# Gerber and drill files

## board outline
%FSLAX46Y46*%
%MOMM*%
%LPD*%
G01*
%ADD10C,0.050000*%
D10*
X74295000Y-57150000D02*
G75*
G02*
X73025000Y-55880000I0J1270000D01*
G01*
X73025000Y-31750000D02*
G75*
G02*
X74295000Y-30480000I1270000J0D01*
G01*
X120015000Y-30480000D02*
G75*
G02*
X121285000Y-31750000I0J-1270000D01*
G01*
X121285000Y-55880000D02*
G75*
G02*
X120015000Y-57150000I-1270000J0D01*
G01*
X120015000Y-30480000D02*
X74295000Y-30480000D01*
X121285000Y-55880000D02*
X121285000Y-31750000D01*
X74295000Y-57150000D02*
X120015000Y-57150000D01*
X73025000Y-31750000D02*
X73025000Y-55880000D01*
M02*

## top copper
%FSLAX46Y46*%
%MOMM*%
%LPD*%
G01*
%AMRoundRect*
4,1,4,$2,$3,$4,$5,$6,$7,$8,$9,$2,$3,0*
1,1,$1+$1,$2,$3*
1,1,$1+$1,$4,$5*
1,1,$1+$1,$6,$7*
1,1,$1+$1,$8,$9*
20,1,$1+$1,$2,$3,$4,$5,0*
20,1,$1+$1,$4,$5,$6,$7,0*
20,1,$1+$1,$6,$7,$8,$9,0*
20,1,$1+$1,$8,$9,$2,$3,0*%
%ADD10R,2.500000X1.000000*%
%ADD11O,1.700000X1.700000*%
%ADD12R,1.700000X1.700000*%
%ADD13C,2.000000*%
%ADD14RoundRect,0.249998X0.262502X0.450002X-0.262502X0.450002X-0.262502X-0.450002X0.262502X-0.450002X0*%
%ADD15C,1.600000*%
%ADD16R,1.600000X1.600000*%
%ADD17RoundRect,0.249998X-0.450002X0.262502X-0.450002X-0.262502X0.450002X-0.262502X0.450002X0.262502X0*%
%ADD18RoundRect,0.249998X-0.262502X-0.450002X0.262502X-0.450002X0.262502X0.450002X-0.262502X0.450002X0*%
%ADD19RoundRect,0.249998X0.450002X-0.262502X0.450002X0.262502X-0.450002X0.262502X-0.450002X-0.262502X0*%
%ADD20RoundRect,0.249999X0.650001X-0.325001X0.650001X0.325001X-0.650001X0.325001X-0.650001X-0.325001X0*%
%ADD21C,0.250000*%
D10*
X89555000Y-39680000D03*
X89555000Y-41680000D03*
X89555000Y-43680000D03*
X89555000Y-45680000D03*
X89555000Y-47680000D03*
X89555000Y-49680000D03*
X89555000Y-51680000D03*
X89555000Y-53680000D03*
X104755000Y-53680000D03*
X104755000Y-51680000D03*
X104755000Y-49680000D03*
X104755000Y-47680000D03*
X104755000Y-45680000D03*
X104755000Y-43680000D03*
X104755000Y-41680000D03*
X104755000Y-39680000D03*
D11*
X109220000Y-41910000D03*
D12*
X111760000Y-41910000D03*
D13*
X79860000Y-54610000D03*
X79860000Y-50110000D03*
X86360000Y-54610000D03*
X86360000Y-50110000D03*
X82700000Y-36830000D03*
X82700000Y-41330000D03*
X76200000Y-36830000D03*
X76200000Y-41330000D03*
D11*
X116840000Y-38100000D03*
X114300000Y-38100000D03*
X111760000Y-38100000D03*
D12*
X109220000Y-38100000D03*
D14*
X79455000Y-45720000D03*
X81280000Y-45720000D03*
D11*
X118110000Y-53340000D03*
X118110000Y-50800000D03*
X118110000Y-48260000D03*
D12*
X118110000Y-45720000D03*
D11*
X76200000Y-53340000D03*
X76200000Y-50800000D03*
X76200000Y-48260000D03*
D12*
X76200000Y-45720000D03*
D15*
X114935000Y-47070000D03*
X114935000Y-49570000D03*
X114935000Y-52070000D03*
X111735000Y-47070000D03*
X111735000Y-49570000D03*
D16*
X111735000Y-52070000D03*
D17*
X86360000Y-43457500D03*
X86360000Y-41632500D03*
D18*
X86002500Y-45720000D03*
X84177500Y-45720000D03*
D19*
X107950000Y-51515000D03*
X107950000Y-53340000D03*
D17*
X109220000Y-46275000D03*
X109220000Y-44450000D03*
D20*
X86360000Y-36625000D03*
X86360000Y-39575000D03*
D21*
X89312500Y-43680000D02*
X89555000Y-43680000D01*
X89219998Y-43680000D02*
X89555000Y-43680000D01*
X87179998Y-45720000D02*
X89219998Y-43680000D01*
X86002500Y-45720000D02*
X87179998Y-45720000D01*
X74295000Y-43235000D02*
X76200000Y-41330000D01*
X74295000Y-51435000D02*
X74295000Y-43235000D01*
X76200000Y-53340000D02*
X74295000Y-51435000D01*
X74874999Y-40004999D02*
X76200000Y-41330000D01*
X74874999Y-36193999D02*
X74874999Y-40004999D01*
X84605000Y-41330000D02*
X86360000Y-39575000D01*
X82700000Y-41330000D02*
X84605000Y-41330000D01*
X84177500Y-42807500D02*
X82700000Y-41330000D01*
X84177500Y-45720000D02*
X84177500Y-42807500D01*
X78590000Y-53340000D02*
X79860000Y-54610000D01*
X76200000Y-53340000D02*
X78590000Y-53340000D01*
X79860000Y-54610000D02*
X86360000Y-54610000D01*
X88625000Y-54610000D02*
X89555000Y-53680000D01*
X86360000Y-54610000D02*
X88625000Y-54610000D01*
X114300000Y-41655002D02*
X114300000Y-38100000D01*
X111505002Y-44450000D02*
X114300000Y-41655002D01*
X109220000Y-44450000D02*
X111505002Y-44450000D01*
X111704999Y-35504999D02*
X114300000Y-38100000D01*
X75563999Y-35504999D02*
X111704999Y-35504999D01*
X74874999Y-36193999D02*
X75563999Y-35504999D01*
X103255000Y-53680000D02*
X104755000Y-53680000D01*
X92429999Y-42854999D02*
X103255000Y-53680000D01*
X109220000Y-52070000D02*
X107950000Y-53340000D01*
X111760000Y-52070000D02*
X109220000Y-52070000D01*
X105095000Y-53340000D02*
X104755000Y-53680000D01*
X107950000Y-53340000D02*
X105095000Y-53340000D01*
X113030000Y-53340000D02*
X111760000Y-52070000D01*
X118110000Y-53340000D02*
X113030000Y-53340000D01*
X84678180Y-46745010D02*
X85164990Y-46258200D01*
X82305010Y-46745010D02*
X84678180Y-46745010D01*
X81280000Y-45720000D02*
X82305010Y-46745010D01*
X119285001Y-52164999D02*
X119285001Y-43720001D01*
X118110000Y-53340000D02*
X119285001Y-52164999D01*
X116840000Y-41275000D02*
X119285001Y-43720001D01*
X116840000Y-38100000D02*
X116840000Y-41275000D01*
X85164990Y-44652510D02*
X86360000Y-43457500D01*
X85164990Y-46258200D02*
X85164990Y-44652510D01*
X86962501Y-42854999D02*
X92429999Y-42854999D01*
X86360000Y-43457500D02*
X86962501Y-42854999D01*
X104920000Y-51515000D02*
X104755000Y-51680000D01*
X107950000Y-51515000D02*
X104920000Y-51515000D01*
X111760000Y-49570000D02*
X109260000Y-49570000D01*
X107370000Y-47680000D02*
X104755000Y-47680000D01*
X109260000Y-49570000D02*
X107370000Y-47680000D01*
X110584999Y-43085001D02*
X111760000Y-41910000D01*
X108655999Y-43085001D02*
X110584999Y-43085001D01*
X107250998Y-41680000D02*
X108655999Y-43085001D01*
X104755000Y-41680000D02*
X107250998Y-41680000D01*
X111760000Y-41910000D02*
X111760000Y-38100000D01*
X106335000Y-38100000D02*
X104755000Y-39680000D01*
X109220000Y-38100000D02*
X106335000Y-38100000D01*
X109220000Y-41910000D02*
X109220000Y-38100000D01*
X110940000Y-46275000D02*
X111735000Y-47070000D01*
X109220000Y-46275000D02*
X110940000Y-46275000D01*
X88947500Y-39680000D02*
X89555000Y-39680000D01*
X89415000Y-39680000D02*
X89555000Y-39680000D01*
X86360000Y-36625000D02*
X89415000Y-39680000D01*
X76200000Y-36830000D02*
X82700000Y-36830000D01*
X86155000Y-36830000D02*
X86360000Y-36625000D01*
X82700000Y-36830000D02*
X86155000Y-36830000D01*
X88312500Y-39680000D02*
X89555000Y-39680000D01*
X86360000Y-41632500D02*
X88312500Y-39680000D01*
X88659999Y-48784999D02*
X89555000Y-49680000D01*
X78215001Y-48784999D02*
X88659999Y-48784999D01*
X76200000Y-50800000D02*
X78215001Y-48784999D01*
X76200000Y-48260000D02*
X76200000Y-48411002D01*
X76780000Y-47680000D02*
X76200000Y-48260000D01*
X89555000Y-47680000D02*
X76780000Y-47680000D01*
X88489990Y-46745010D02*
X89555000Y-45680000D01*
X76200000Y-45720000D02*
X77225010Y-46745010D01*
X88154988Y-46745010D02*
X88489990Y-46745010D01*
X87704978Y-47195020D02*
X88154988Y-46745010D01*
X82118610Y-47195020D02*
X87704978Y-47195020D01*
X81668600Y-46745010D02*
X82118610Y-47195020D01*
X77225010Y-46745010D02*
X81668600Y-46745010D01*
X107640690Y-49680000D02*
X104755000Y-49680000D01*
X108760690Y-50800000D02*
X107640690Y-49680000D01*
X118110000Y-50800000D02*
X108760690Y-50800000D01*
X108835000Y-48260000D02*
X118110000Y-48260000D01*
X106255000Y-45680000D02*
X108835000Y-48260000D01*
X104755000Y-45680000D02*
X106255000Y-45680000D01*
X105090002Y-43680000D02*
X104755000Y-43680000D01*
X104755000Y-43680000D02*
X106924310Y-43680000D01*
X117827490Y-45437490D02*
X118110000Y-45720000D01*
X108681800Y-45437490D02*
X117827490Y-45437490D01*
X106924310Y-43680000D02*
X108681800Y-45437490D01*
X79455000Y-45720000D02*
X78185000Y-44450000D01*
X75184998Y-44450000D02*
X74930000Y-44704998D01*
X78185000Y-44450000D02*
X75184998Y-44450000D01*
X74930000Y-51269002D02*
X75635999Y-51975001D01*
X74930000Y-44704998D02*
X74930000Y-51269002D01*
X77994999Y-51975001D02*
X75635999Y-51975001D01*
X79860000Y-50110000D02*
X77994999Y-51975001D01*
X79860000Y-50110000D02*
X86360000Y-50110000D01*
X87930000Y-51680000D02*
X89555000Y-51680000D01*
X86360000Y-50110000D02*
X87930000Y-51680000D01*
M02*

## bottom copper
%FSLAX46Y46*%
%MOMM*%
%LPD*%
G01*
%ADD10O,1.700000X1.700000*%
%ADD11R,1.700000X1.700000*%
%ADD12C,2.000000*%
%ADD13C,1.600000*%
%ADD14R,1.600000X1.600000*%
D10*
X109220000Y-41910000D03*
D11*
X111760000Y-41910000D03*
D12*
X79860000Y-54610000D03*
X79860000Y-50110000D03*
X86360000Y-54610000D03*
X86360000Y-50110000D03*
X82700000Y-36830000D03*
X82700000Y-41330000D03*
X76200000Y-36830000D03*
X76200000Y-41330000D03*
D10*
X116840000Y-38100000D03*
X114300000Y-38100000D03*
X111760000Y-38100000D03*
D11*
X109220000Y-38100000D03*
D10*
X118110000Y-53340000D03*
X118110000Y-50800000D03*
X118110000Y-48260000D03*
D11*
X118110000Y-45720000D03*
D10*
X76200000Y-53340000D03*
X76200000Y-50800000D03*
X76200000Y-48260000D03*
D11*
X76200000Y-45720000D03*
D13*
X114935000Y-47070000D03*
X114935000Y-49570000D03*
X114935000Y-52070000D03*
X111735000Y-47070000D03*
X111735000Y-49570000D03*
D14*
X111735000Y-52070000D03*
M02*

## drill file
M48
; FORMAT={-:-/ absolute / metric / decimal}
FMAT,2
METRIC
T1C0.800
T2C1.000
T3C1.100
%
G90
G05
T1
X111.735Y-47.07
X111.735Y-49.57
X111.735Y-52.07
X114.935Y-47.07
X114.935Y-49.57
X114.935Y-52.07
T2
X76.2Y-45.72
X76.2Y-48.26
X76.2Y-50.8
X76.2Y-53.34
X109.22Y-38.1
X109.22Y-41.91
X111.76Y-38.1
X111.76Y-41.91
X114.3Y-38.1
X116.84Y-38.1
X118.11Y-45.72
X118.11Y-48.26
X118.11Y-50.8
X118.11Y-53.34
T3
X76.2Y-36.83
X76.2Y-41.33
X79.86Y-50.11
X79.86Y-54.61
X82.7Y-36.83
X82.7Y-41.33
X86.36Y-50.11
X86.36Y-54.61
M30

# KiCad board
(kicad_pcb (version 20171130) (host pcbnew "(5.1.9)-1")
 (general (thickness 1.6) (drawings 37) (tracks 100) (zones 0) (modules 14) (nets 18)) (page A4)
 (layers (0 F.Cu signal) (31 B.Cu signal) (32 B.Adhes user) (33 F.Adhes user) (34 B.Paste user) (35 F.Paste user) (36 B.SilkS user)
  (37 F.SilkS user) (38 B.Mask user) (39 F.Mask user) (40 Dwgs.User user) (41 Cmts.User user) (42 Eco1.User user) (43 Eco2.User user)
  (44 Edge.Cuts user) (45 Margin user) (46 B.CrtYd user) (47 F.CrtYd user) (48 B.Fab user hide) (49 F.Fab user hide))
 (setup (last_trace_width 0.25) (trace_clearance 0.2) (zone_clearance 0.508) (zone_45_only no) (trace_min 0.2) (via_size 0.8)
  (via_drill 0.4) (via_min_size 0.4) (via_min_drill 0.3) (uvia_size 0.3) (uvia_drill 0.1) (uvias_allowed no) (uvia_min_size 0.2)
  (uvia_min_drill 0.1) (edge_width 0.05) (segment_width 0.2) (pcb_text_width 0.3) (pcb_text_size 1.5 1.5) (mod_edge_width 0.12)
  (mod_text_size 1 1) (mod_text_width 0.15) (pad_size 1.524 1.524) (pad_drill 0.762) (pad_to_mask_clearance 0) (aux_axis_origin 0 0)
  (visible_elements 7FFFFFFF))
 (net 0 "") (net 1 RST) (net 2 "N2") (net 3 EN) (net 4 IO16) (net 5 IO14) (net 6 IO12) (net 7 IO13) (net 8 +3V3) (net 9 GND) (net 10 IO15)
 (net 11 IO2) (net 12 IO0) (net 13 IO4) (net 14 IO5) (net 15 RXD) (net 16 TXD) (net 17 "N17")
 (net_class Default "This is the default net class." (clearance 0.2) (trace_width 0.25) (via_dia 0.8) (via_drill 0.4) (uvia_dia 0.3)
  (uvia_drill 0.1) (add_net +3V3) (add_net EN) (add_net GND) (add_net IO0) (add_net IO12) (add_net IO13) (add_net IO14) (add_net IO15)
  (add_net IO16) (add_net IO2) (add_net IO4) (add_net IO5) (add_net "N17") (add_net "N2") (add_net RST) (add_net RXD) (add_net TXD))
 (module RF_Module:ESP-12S (layer F.Cu) (at 97.155 43.18)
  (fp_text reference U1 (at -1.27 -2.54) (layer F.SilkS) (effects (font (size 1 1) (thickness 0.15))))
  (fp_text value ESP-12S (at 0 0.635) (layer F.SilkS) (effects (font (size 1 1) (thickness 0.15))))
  (pad 1 smd rect (at -7.6 -3.5) (size 2.5 1) (layers F.Cu F.Paste F.Mask) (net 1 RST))
  (pad 2 smd rect (at -7.6 -1.5) (size 2.5 1) (layers F.Cu F.Paste F.Mask) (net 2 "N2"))
  (pad 3 smd rect (at -7.6 0.5) (size 2.5 1) (layers F.Cu F.Paste F.Mask) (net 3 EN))
  (pad 4 smd rect (at -7.6 2.5) (size 2.5 1) (layers F.Cu F.Paste F.Mask) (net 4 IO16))
  (pad 5 smd rect (at -7.6 4.5) (size 2.5 1) (layers F.Cu F.Paste F.Mask) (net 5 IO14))
  (pad 6 smd rect (at -7.6 6.5) (size 2.5 1) (layers F.Cu F.Paste F.Mask) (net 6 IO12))
  (pad 7 smd rect (at -7.6 8.5) (size 2.5 1) (layers F.Cu F.Paste F.Mask) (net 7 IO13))
  (pad 8 smd rect (at -7.6 10.5) (size 2.5 1) (layers F.Cu F.Paste F.Mask) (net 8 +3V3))
  (pad 9 smd rect (at 7.6 10.5) (size 2.5 1) (layers F.Cu F.Paste F.Mask) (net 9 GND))
  (pad 10 smd rect (at 7.6 8.5) (size 2.5 1) (layers F.Cu F.Paste F.Mask) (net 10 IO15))
  (pad 11 smd rect (at 7.6 6.5) (size 2.5 1) (layers F.Cu F.Paste F.Mask) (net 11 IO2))
  (pad 12 smd rect (at 7.6 4.5) (size 2.5 1) (layers F.Cu F.Paste F.Mask) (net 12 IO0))
  (pad 13 smd rect (at 7.6 2.5) (size 2.5 1) (layers F.Cu F.Paste F.Mask) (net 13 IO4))
  (pad 14 smd rect (at 7.6 0.5) (size 2.5 1) (layers F.Cu F.Paste F.Mask) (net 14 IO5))
  (pad 15 smd rect (at 7.6 -1.5) (size 2.5 1) (layers F.Cu F.Paste F.Mask) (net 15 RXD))
  (pad 16 smd rect (at 7.6 -3.5) (size 2.5 1) (layers F.Cu F.Paste F.Mask) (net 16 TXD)))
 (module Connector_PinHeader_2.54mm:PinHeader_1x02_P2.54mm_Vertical (layer B.Cu) (at 111.76 41.91 90)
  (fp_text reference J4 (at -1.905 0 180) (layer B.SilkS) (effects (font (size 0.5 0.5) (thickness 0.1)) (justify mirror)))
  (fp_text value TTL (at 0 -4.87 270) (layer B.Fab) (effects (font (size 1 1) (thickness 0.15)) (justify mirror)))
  (pad 2 thru_hole oval (at 0 -2.54 90) (size 1.7 1.7) (drill 1) (layers *.Cu *.Mask) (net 16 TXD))
  (pad 1 thru_hole rect (at 0 0 90) (size 1.7 1.7) (drill 1) (layers *.Cu *.Mask) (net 15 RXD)))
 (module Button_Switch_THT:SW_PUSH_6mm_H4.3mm (layer F.Cu) (at 86.36 54.61 180)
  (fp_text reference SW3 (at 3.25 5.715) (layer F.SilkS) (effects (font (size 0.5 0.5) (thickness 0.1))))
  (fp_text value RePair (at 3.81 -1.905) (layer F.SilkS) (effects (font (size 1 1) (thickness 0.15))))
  (pad 1 thru_hole circle (at 6.5 0 270) (size 2 2) (drill 1.1) (layers *.Cu *.Mask) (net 8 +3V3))
  (pad 2 thru_hole circle (at 6.5 4.5 270) (size 2 2) (drill 1.1) (layers *.Cu *.Mask) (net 7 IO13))
  (pad 1 thru_hole circle (at 0 0 270) (size 2 2) (drill 1.1) (layers *.Cu *.Mask) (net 8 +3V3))
  (pad 2 thru_hole circle (at 0 4.5 270) (size 2 2) (drill 1.1) (layers *.Cu *.Mask) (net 7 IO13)))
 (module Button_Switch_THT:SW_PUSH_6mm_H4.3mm (layer F.Cu) (at 76.2 36.83)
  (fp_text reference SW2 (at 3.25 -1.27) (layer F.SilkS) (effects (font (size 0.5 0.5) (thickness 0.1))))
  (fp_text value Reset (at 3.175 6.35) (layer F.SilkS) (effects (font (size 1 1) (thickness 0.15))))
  (pad 1 thru_hole circle (at 6.5 0 90) (size 2 2) (drill 1.1) (layers *.Cu *.Mask) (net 1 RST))
  (pad 2 thru_hole circle (at 6.5 4.5 90) (size 2 2) (drill 1.1) (layers *.Cu *.Mask) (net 8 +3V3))
  (pad 1 thru_hole circle (at 0 0 90) (size 2 2) (drill 1.1) (layers *.Cu *.Mask) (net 1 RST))
  (pad 2 thru_hole circle (at 0 4.5 90) (size 2 2) (drill 1.1) (layers *.Cu *.Mask) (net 8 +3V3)))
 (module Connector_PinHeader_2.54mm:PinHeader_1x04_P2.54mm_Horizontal (layer F.Cu) (at 109.22 38.1 90)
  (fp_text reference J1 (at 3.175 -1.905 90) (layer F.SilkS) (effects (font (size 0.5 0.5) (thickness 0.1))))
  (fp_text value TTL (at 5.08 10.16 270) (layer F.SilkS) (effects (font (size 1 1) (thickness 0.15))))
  (pad 4 thru_hole oval (at 0 7.62 90) (size 1.7 1.7) (drill 1) (layers *.Cu *.Mask) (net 9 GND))
  (pad 3 thru_hole oval (at 0 5.08 90) (size 1.7 1.7) (drill 1) (layers *.Cu *.Mask) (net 8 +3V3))
  (pad 2 thru_hole oval (at 0 2.54 90) (size 1.7 1.7) (drill 1) (layers *.Cu *.Mask) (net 15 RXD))
  (pad 1 thru_hole rect (at 0 0 90) (size 1.7 1.7) (drill 1) (layers *.Cu *.Mask) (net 16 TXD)))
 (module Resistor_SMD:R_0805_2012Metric (layer F.Cu) (at 80.3675 45.72 180)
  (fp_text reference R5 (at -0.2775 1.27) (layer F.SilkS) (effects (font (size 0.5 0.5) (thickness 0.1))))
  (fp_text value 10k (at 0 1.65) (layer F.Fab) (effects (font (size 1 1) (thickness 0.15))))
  (pad 2 smd roundrect (at 0.9125 0 180) (size 1.025 1.4) (layers F.Cu F.Paste F.Mask) (roundrect_rratio 0.2439004878048781) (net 7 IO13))
  (pad 1 smd roundrect (at -0.9125 0 180) (size 1.025 1.4) (layers F.Cu F.Paste F.Mask) (roundrect_rratio 0.2439004878048781) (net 9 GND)))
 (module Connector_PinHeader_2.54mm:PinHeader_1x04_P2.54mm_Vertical (layer B.Cu) (at 118.11 45.72 180)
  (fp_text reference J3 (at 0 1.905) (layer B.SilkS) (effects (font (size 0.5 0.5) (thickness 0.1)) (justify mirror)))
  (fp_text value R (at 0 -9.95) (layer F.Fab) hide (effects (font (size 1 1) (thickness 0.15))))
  (pad 4 thru_hole oval (at 0 -7.62 180) (size 1.7 1.7) (drill 1) (layers *.Cu *.Mask) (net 9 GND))
  (pad 3 thru_hole oval (at 0 -5.08 180) (size 1.7 1.7) (drill 1) (layers *.Cu *.Mask) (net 11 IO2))
  (pad 2 thru_hole oval (at 0 -2.54 180) (size 1.7 1.7) (drill 1) (layers *.Cu *.Mask) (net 13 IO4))
  (pad 1 thru_hole rect (at 0 0 180) (size 1.7 1.7) (drill 1) (layers *.Cu *.Mask) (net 14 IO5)))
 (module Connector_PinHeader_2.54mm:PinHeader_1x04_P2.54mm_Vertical (layer B.Cu) (at 76.2 45.72 180)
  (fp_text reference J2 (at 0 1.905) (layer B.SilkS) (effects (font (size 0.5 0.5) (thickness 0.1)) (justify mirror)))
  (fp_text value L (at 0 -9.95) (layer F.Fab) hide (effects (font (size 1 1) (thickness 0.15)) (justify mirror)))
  (pad 4 thru_hole oval (at 0 -7.62 180) (size 1.7 1.7) (drill 1) (layers *.Cu *.Mask) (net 8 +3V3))
  (pad 3 thru_hole oval (at 0 -5.08 180) (size 1.7 1.7) (drill 1) (layers *.Cu *.Mask) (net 6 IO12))
  (pad 2 thru_hole oval (at 0 -2.54 180) (size 1.7 1.7) (drill 1) (layers *.Cu *.Mask) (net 5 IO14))
  (pad 1 thru_hole rect (at 0 0 180) (size 1.7 1.7) (drill 1) (layers *.Cu *.Mask) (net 4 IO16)))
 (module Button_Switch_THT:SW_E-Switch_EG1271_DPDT (layer F.Cu) (at 111.735 52.07 90)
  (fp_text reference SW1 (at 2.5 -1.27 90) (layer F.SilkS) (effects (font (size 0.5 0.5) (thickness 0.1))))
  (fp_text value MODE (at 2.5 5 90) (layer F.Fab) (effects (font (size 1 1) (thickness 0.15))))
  (pad 6 thru_hole circle (at 5 3.2 90) (size 1.6 1.6) (drill 0.8) (layers *.Cu *.Mask))
  (pad 5 thru_hole circle (at 2.5 3.2 90) (size 1.6 1.6) (drill 0.8) (layers *.Cu *.Mask))
  (pad 4 thru_hole circle (at 0 3.2 90) (size 1.6 1.6) (drill 0.8) (layers *.Cu *.Mask))
  (pad 3 thru_hole circle (at 5 0 90) (size 1.6 1.6) (drill 0.8) (layers *.Cu *.Mask) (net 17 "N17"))
  (pad 2 thru_hole circle (at 2.5 0 90) (size 1.6 1.6) (drill 0.8) (layers *.Cu *.Mask) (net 12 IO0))
  (pad 1 thru_hole rect (at 0 0 90) (size 1.6 1.6) (drill 0.8) (layers *.Cu *.Mask) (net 9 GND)))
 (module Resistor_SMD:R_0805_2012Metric (layer F.Cu) (at 86.36 42.545 270)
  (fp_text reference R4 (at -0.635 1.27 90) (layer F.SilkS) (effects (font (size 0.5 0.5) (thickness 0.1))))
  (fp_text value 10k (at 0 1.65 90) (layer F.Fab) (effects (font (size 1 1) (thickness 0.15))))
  (pad 2 smd roundrect (at 0.9125 0 270) (size 1.025 1.4) (layers F.Cu F.Paste F.Mask) (roundrect_rratio 0.2439004878048781) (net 9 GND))
  (pad 1 smd roundrect (at -0.9125 0 270) (size 1.025 1.4) (layers F.Cu F.Paste F.Mask) (roundrect_rratio 0.2439004878048781) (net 1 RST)))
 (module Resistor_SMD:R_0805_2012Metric (layer F.Cu) (at 85.09 45.72)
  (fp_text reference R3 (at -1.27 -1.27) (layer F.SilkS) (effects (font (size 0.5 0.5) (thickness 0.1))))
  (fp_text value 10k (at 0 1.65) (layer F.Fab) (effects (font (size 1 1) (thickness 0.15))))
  (pad 2 smd roundrect (at 0.9125 0) (size 1.025 1.4) (layers F.Cu F.Paste F.Mask) (roundrect_rratio 0.2439004878048781) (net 3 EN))
  (pad 1 smd roundrect (at -0.9125 0) (size 1.025 1.4) (layers F.Cu F.Paste F.Mask) (roundrect_rratio 0.2439004878048781) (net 8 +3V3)))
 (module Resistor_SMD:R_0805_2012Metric (layer F.Cu) (at 107.95 52.4275 90)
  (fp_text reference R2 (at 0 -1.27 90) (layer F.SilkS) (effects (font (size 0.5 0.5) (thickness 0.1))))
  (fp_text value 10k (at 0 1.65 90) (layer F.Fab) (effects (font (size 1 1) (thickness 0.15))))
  (pad 2 smd roundrect (at 0.9125 0 90) (size 1.025 1.4) (layers F.Cu F.Paste F.Mask) (roundrect_rratio 0.2439004878048781) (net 10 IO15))
  (pad 1 smd roundrect (at -0.9125 0 90) (size 1.025 1.4) (layers F.Cu F.Paste F.Mask) (roundrect_rratio 0.2439004878048781) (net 9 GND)))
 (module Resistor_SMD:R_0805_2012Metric (layer F.Cu) (at 109.22 45.3625 270)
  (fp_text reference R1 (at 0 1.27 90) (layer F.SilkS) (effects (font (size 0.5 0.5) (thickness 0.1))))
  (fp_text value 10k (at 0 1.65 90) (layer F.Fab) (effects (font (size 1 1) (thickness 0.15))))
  (pad 2 smd roundrect (at 0.9125 0 270) (size 1.025 1.4) (layers F.Cu F.Paste F.Mask) (roundrect_rratio 0.2439004878048781) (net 17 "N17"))
  (pad 1 smd roundrect (at -0.9125 0 270) (size 1.025 1.4) (layers F.Cu F.Paste F.Mask) (roundrect_rratio 0.2439004878048781) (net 8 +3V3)))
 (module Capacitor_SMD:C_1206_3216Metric (layer F.Cu) (at 86.36 38.1 90)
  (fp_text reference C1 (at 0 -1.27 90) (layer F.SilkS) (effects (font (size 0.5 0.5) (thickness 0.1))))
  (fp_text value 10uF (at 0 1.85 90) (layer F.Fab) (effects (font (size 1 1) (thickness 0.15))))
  (pad 2 smd roundrect (at 1.475 0 90) (size 1.15 1.8) (layers F.Cu F.Paste F.Mask) (roundrect_rratio 0.2173904347826087) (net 1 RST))
  (pad 1 smd roundrect (at -1.475 0 90) (size 1.15 1.8) (layers F.Cu F.Paste F.Mask) (roundrect_rratio 0.2173904347826087) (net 8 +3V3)))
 (gr_arc (start 74.295 55.88) (end 73.025 55.88) (angle -90) (layer Edge.Cuts) (width 0.05))
 (gr_arc (start 74.295 31.75) (end 74.295 30.48) (angle -90) (layer Edge.Cuts) (width 0.05))
 (gr_arc (start 120.015 31.75) (end 121.285 31.75) (angle -90) (layer Edge.Cuts) (width 0.05))
 (gr_arc (start 120.015 55.88) (end 120.015 57.15) (angle -90) (layer Edge.Cuts) (width 0.05))
 (gr_line (start 120.015 30.48) (end 74.295 30.48) (layer Edge.Cuts) (width 0.05))
 (gr_line (start 121.285 55.88) (end 121.285 31.75) (layer Edge.Cuts) (width 0.05))
 (gr_line (start 74.295 57.15) (end 120.015 57.15) (layer Edge.Cuts) (width 0.05))
 (gr_line (start 73.025 31.75) (end 73.025 55.88) (layer Edge.Cuts) (width 0.05))
 (segment (start 89.3125 43.68) (end 89.555 43.68) (width 0.25) (layer F.Cu) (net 3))
 (segment (start 89.219998 43.68) (end 89.555 43.68) (width 0.25) (layer F.Cu) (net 3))
 (segment (start 87.179998 45.72) (end 89.219998 43.68) (width 0.25) (layer F.Cu) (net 3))
 (segment (start 86.0025 45.72) (end 87.179998 45.72) (width 0.25) (layer F.Cu) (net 3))
 (segment (start 74.295 43.235) (end 76.2 41.33) (width 0.25) (layer F.Cu) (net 8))
 (segment (start 74.295 51.435) (end 74.295 43.235) (width 0.25) (layer F.Cu) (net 8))
 (segment (start 76.2 53.34) (end 74.295 51.435) (width 0.25) (layer F.Cu) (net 8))
 (segment (start 74.874999 40.004999) (end 76.2 41.33) (width 0.25) (layer F.Cu) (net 8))
 (segment (start 74.874999 36.193999) (end 74.874999 40.004999) (width 0.25) (layer F.Cu) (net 8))
 (segment (start 84.605 41.33) (end 86.36 39.575) (width 0.25) (layer F.Cu) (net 8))
 (segment (start 82.7 41.33) (end 84.605 41.33) (width 0.25) (layer F.Cu) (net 8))
 (segment (start 84.1775 42.8075) (end 82.7 41.33) (width 0.25) (layer F.Cu) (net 8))
 (segment (start 84.1775 45.72) (end 84.1775 42.8075) (width 0.25) (layer F.Cu) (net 8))
 (segment (start 78.59 53.34) (end 79.86 54.61) (width 0.25) (layer F.Cu) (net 8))
 (segment (start 76.2 53.34) (end 78.59 53.34) (width 0.25) (layer F.Cu) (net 8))
 (segment (start 79.86 54.61) (end 86.36 54.61) (width 0.25) (layer F.Cu) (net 8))
 (segment (start 88.625 54.61) (end 89.555 53.68) (width 0.25) (layer F.Cu) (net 8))
 (segment (start 86.36 54.61) (end 88.625 54.61) (width 0.25) (layer F.Cu) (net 8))
 (segment (start 114.3 41.655002) (end 114.3 38.1) (width 0.25) (layer F.Cu) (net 8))
 (segment (start 111.505002 44.45) (end 114.3 41.655002) (width 0.25) (layer F.Cu) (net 8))
 (segment (start 109.22 44.45) (end 111.505002 44.45) (width 0.25) (layer F.Cu) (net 8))
 (segment (start 111.704999 35.504999) (end 114.3 38.1) (width 0.25) (layer F.Cu) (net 8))
 (segment (start 75.563999 35.504999) (end 111.704999 35.504999) (width 0.25) (layer F.Cu) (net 8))
 (segment (start 74.874999 36.193999) (end 75.563999 35.504999) (width 0.25) (layer F.Cu) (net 8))
 (segment (start 103.255 53.68) (end 104.755 53.68) (width 0.25) (layer F.Cu) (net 9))
 (segment (start 92.429999 42.854999) (end 103.255 53.68) (width 0.25) (layer F.Cu) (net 9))
 (segment (start 109.22 52.07) (end 107.95 53.34) (width 0.25) (layer F.Cu) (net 9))
 (segment (start 111.76 52.07) (end 109.22 52.07) (width 0.25) (layer F.Cu) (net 9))
 (segment (start 105.095 53.34) (end 104.755 53.68) (width 0.25) (layer F.Cu) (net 9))
 (segment (start 107.95 53.34) (end 105.095 53.34) (width 0.25) (layer F.Cu) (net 9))
 (segment (start 113.03 53.34) (end 111.76 52.07) (width 0.25) (layer F.Cu) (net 9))
 (segment (start 118.11 53.34) (end 113.03 53.34) (width 0.25) (layer F.Cu) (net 9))
 (segment (start 84.67818 46.74501) (end 85.16499 46.2582) (width 0.25) (layer F.Cu) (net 9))
 (segment (start 82.30501 46.74501) (end 84.67818 46.74501) (width 0.25) (layer F.Cu) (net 9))
 (segment (start 81.28 45.72) (end 82.30501 46.74501) (width 0.25) (layer F.Cu) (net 9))
 (segment (start 119.285001 52.164999) (end 119.285001 43.720001) (width 0.25) (layer F.Cu) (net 9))
 (segment (start 118.11 53.34) (end 119.285001 52.164999) (width 0.25) (layer F.Cu) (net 9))
 (segment (start 116.84 41.275) (end 119.285001 43.720001) (width 0.25) (layer F.Cu) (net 9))
 (segment (start 116.84 38.1) (end 116.84 41.275) (width 0.25) (layer F.Cu) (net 9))
 (segment (start 85.16499 44.65251) (end 86.36 43.4575) (width 0.25) (layer F.Cu) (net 9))
 (segment (start 85.16499 46.2582) (end 85.16499 44.65251) (width 0.25) (layer F.Cu) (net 9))
 (segment (start 86.962501 42.854999) (end 92.429999 42.854999) (width 0.25) (layer F.Cu) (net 9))
 (segment (start 86.36 43.4575) (end 86.962501 42.854999) (width 0.25) (layer F.Cu) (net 9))
 (segment (start 104.92 51.515) (end 104.755 51.68) (width 0.25) (layer F.Cu) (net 10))
 (segment (start 107.95 51.515) (end 104.92 51.515) (width 0.25) (layer F.Cu) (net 10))
 (segment (start 111.76 49.57) (end 109.26 49.57) (width 0.25) (layer F.Cu) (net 12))
 (segment (start 107.37 47.68) (end 104.755 47.68) (width 0.25) (layer F.Cu) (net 12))
 (segment (start 109.26 49.57) (end 107.37 47.68) (width 0.25) (layer F.Cu) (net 12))
 (segment (start 110.584999 43.085001) (end 111.76 41.91) (width 0.25) (layer F.Cu) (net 15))
 (segment (start 108.655999 43.085001) (end 110.584999 43.085001) (width 0.25) (layer F.Cu) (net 15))
 (segment (start 107.250998 41.68) (end 108.655999 43.085001) (width 0.25) (layer F.Cu) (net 15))
 (segment (start 104.755 41.68) (end 107.250998 41.68) (width 0.25) (layer F.Cu) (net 15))
 (segment (start 111.76 41.91) (end 111.76 38.1) (width 0.25) (layer F.Cu) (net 15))
 (segment (start 106.335 38.1) (end 104.755 39.68) (width 0.25) (layer F.Cu) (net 16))
 (segment (start 109.22 38.1) (end 106.335 38.1) (width 0.25) (layer F.Cu) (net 16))
 (segment (start 109.22 41.91) (end 109.22 38.1) (width 0.25) (layer F.Cu) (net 16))
 (segment (start 110.94 46.275) (end 111.735 47.07) (width 0.25) (layer F.Cu) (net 17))
 (segment (start 109.22 46.275) (end 110.94 46.275) (width 0.25) (layer F.Cu) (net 17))
 (segment (start 88.9475 39.68) (end 89.555 39.68) (width 0.25) (layer F.Cu) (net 1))
 (segment (start 89.415 39.68) (end 89.555 39.68) (width 0.25) (layer F.Cu) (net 1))
 (segment (start 86.36 36.625) (end 89.415 39.68) (width 0.25) (layer F.Cu) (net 1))
 (segment (start 76.2 36.83) (end 82.7 36.83) (width 0.25) (layer F.Cu) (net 1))
 (segment (start 86.155 36.83) (end 86.36 36.625) (width 0.25) (layer F.Cu) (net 1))
 (segment (start 82.7 36.83) (end 86.155 36.83) (width 0.25) (layer F.Cu) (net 1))
 (segment (start 88.3125 39.68) (end 89.555 39.68) (width 0.25) (layer F.Cu) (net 1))
 (segment (start 86.36 41.6325) (end 88.3125 39.68) (width 0.25) (layer F.Cu) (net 1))
 (segment (start 88.659999 48.784999) (end 89.555 49.68) (width 0.25) (layer F.Cu) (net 6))
 (segment (start 78.215001 48.784999) (end 88.659999 48.784999) (width 0.25) (layer F.Cu) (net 6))
 (segment (start 76.2 50.8) (end 78.215001 48.784999) (width 0.25) (layer F.Cu) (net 6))
 (segment (start 76.2 48.26) (end 76.2 48.411002) (width 0.25) (layer F.Cu) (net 5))
 (segment (start 76.78 47.68) (end 76.2 48.26) (width 0.25) (layer F.Cu) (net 5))
 (segment (start 89.555 47.68) (end 76.78 47.68) (width 0.25) (layer F.Cu) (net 5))
 (segment (start 88.48999 46.74501) (end 89.555 45.68) (width 0.25) (layer F.Cu) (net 4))
 (segment (start 76.2 45.72) (end 77.22501 46.74501) (width 0.25) (layer F.Cu) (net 4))
 (segment (start 88.154988 46.74501) (end 88.48999 46.74501) (width 0.25) (layer F.Cu) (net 4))
 (segment (start 87.704978 47.19502) (end 88.154988 46.74501) (width 0.25) (layer F.Cu) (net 4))
 (segment (start 82.11861 47.19502) (end 87.704978 47.19502) (width 0.25) (layer F.Cu) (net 4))
 (segment (start 81.6686 46.74501) (end 82.11861 47.19502) (width 0.25) (layer F.Cu) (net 4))
 (segment (start 77.22501 46.74501) (end 81.6686 46.74501) (width 0.25) (layer F.Cu) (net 4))
 (segment (start 107.64069 49.68) (end 104.755 49.68) (width 0.25) (layer F.Cu) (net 11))
 (segment (start 108.76069 50.8) (end 107.64069 49.68) (width 0.25) (layer F.Cu) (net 11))
 (segment (start 118.11 50.8) (end 108.76069 50.8) (width 0.25) (layer F.Cu) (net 11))
 (segment (start 108.835 48.26) (end 118.11 48.26) (width 0.25) (layer F.Cu) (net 13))
 (segment (start 106.255 45.68) (end 108.835 48.26) (width 0.25) (layer F.Cu) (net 13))
 (segment (start 104.755 45.68) (end 106.255 45.68) (width 0.25) (layer F.Cu) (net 13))
 (segment (start 105.090002 43.68) (end 104.755 43.68) (width 0.25) (layer F.Cu) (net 14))
 (segment (start 104.755 43.68) (end 106.92431 43.68) (width 0.25) (layer F.Cu) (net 14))
 (segment (start 117.82749 45.43749) (end 118.11 45.72) (width 0.25) (layer F.Cu) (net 14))
 (segment (start 108.6818 45.43749) (end 117.82749 45.43749) (width 0.25) (layer F.Cu) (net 14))
 (segment (start 106.92431 43.68) (end 108.6818 45.43749) (width 0.25) (layer F.Cu) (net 14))
 (segment (start 79.455 45.72) (end 78.185 44.45) (width 0.25) (layer F.Cu) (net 7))
 (segment (start 75.184998 44.45) (end 74.93 44.704998) (width 0.25) (layer F.Cu) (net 7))
 (segment (start 78.185 44.45) (end 75.184998 44.45) (width 0.25) (layer F.Cu) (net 7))
 (segment (start 74.93 51.269002) (end 75.635999 51.975001) (width 0.25) (layer F.Cu) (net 7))
 (segment (start 74.93 44.704998) (end 74.93 51.269002) (width 0.25) (layer F.Cu) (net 7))
 (segment (start 77.994999 51.975001) (end 75.635999 51.975001) (width 0.25) (layer F.Cu) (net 7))
 (segment (start 79.86 50.11) (end 77.994999 51.975001) (width 0.25) (layer F.Cu) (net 7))
 (segment (start 79.86 50.11) (end 86.36 50.11) (width 0.25) (layer F.Cu) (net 7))
 (segment (start 87.93 51.68) (end 89.555 51.68) (width 0.25) (layer F.Cu) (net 7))
 (segment (start 86.36 50.11) (end 87.93 51.68) (width 0.25) (layer F.Cu) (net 7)))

